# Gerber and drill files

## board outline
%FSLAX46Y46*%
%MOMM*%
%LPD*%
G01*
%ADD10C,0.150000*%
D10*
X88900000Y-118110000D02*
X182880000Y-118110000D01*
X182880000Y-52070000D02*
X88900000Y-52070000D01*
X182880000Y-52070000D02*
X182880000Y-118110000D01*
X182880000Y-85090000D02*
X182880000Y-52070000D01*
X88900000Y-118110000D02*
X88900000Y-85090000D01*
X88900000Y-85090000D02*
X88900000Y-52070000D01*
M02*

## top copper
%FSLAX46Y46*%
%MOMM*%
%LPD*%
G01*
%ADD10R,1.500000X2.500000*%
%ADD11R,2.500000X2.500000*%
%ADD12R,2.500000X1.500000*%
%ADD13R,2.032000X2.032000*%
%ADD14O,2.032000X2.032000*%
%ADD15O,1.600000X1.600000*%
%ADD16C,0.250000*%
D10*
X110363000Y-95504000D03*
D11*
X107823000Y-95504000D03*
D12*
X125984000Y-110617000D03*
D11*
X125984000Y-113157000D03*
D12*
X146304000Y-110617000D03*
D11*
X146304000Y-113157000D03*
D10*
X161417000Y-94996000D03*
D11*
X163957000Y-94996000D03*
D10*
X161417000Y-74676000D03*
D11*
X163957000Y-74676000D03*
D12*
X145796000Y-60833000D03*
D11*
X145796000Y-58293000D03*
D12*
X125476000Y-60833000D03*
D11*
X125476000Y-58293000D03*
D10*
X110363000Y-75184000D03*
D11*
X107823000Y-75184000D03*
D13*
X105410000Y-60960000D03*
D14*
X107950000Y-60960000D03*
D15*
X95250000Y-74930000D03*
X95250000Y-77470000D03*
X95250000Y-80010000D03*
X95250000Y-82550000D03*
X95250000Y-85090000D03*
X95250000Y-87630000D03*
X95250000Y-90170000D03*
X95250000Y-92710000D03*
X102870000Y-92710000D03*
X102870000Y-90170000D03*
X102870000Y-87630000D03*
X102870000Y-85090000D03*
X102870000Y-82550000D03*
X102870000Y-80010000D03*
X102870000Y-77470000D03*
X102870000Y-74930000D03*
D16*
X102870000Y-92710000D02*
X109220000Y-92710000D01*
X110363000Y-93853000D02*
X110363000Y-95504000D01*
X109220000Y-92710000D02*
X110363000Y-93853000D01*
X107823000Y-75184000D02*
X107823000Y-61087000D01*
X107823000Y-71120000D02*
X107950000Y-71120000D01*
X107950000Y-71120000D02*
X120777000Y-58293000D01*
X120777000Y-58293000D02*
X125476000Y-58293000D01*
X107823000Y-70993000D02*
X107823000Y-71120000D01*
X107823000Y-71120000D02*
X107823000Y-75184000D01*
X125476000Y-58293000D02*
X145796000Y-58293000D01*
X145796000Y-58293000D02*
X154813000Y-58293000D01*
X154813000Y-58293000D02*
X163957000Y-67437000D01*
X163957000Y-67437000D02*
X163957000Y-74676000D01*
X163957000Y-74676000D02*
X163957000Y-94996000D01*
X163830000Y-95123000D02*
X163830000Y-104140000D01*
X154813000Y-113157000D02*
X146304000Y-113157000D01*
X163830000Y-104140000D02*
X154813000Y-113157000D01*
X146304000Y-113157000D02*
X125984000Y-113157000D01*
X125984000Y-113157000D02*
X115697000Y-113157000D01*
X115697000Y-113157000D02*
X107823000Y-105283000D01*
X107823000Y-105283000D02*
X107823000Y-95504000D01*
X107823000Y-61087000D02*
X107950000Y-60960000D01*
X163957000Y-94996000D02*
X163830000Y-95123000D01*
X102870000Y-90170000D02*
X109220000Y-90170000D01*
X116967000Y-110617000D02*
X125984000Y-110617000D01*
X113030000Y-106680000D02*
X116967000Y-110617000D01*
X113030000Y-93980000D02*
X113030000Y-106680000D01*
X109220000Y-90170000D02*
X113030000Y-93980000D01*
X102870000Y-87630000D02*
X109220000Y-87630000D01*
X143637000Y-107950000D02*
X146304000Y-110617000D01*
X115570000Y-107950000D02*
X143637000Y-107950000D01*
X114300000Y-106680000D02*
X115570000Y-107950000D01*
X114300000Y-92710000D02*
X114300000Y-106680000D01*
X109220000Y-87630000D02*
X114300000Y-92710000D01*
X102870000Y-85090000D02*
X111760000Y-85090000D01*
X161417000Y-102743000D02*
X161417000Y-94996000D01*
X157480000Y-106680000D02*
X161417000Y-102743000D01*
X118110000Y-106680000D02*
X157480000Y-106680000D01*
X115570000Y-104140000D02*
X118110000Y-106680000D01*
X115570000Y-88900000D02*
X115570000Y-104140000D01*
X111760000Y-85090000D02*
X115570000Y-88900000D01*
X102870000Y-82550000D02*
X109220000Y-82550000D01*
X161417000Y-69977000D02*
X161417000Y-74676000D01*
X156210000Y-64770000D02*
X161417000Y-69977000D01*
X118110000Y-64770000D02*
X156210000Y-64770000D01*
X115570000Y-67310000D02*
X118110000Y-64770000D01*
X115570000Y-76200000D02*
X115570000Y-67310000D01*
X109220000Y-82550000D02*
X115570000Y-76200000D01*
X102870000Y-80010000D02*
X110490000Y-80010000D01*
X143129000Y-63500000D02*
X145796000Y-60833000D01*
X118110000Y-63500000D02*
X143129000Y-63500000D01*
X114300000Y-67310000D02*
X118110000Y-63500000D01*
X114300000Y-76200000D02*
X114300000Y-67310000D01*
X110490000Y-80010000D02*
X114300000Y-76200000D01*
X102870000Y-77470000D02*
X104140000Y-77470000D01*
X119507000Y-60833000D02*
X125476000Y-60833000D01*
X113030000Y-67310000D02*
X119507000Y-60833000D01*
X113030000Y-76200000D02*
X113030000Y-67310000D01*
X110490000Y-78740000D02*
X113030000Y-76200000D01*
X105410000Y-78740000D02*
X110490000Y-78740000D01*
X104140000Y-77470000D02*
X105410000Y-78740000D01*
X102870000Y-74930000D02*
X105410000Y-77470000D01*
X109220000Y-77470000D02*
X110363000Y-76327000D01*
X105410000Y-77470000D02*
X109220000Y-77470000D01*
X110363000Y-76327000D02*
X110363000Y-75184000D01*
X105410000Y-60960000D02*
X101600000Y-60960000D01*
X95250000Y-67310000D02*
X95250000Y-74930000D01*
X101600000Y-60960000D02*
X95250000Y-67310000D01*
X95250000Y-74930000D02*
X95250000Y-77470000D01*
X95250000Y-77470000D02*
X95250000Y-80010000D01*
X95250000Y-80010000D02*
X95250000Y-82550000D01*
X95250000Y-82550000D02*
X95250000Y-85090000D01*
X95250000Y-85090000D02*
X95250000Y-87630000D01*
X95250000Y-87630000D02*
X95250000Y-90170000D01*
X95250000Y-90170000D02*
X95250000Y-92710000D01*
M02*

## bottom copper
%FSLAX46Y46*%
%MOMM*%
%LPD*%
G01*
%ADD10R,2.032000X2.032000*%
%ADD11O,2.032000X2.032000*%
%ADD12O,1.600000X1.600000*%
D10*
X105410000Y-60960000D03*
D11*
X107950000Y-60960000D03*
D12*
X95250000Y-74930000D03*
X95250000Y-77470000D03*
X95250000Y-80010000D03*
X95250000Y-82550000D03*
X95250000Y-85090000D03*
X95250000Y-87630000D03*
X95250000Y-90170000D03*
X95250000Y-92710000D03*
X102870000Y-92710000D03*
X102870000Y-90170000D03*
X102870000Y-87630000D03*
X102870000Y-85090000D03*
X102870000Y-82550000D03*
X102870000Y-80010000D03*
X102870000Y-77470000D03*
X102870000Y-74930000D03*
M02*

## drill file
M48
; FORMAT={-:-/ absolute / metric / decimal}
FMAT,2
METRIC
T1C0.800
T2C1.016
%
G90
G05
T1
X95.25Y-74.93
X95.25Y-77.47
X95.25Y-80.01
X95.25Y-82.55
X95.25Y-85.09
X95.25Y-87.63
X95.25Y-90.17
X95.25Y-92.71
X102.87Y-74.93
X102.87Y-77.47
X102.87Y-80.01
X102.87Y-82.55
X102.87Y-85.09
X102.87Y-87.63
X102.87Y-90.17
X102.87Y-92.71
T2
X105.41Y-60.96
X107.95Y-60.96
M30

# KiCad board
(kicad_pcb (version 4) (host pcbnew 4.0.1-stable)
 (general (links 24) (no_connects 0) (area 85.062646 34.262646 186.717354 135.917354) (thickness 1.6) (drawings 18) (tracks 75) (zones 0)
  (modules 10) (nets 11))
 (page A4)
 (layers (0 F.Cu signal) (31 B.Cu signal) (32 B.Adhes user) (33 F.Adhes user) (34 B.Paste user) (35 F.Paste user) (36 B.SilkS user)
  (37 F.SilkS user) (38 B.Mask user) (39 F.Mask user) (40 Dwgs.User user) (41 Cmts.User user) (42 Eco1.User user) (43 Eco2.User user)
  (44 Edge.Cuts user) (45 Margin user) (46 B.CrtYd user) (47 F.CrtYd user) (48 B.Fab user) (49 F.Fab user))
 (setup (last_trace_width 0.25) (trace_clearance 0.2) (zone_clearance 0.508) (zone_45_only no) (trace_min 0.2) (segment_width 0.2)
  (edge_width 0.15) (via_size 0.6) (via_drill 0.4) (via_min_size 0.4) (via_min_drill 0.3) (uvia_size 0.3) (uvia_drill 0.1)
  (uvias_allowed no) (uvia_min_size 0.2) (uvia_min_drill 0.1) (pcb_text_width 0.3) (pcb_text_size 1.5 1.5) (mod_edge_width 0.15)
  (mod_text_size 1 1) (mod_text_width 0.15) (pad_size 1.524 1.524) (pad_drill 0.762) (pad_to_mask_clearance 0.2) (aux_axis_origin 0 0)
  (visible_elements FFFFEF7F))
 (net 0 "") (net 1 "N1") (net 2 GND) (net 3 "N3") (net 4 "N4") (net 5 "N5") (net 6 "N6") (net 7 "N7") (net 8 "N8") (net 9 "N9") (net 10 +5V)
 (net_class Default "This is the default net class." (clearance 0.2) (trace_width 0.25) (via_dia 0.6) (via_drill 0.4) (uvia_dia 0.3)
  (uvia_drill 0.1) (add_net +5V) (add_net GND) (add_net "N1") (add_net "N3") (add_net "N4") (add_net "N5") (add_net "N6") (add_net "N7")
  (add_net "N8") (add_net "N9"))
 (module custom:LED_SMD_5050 (layer F.Cu) (at 109.22 91.44)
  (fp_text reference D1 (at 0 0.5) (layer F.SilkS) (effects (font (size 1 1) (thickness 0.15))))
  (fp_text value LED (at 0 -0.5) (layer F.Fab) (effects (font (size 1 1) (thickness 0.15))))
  (pad 2 smd rect (at 1.143 4.064) (size 1.5 2.5) (layers F.Cu F.Paste F.Mask) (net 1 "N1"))
  (pad 1 smd rect (at -1.397 4.064) (size 2.5 2.5) (layers F.Cu F.Paste F.Mask) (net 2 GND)))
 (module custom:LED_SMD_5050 (layer F.Cu) (at 121.92 111.76 90)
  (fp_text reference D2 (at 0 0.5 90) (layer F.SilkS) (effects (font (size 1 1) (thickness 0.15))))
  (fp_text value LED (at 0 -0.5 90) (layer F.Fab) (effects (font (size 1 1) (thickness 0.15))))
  (pad 2 smd rect (at 1.143 4.064 90) (size 1.5 2.5) (layers F.Cu F.Paste F.Mask) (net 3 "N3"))
  (pad 1 smd rect (at -1.397 4.064 90) (size 2.5 2.5) (layers F.Cu F.Paste F.Mask) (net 2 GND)))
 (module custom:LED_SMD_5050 (layer F.Cu) (at 142.24 111.76 90)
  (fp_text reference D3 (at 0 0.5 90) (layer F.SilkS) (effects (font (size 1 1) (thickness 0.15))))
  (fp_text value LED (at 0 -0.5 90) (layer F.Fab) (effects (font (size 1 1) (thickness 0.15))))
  (pad 2 smd rect (at 1.143 4.064 90) (size 1.5 2.5) (layers F.Cu F.Paste F.Mask) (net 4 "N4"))
  (pad 1 smd rect (at -1.397 4.064 90) (size 2.5 2.5) (layers F.Cu F.Paste F.Mask) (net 2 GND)))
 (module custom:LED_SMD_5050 (layer F.Cu) (at 162.56 99.06 180)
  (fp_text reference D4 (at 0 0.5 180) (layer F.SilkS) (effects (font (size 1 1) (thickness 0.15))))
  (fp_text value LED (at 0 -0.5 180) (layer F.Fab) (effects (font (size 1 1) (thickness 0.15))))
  (pad 2 smd rect (at 1.143 4.064 180) (size 1.5 2.5) (layers F.Cu F.Paste F.Mask) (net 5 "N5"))
  (pad 1 smd rect (at -1.397 4.064 180) (size 2.5 2.5) (layers F.Cu F.Paste F.Mask) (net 2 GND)))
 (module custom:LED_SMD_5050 (layer F.Cu) (at 162.56 78.74 180)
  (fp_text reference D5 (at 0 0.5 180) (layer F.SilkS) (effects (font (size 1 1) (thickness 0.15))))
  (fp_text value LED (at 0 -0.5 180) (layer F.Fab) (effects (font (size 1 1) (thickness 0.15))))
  (pad 2 smd rect (at 1.143 4.064 180) (size 1.5 2.5) (layers F.Cu F.Paste F.Mask) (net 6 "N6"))
  (pad 1 smd rect (at -1.397 4.064 180) (size 2.5 2.5) (layers F.Cu F.Paste F.Mask) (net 2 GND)))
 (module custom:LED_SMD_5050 (layer F.Cu) (at 149.86 59.69 270)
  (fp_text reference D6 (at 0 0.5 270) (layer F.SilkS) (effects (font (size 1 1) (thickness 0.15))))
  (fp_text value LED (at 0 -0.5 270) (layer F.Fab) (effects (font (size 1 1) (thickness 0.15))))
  (pad 2 smd rect (at 1.143 4.064 270) (size 1.5 2.5) (layers F.Cu F.Paste F.Mask) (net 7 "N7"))
  (pad 1 smd rect (at -1.397 4.064 270) (size 2.5 2.5) (layers F.Cu F.Paste F.Mask) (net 2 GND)))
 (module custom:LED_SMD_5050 (layer F.Cu) (at 129.54 59.69 270)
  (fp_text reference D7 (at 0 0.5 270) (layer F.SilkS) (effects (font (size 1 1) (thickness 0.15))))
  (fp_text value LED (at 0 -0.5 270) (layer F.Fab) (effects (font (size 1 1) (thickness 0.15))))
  (pad 2 smd rect (at 1.143 4.064 270) (size 1.5 2.5) (layers F.Cu F.Paste F.Mask) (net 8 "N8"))
  (pad 1 smd rect (at -1.397 4.064 270) (size 2.5 2.5) (layers F.Cu F.Paste F.Mask) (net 2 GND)))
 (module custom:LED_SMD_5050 (layer F.Cu) (at 109.22 71.12)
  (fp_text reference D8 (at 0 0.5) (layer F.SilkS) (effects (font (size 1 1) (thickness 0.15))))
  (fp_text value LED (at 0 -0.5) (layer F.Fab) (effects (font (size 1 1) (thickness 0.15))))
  (pad 2 smd rect (at 1.143 4.064) (size 1.5 2.5) (layers F.Cu F.Paste F.Mask) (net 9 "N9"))
  (pad 1 smd rect (at -1.397 4.064) (size 2.5 2.5) (layers F.Cu F.Paste F.Mask) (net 2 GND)))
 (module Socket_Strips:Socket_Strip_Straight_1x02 (layer F.Cu) (at 105.41 60.96)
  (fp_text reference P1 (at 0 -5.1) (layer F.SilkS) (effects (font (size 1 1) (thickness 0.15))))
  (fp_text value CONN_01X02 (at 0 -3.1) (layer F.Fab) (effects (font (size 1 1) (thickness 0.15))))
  (pad 1 thru_hole rect (at 0 0) (size 2.032 2.032) (drill 1.016) (layers *.Cu *.Mask F.SilkS) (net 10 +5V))
  (pad 2 thru_hole oval (at 2.54 0) (size 2.032 2.032) (drill 1.016) (layers *.Cu *.Mask F.SilkS) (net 2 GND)))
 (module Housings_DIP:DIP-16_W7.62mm (layer F.Cu) (at 95.25 74.93)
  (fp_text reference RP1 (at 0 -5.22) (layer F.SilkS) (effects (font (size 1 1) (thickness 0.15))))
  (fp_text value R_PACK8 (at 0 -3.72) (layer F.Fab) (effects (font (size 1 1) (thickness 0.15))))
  (pad 1 thru_hole oval (at 0 0) (size 1.6 1.6) (drill 0.8) (layers *.Cu *.Mask F.SilkS) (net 10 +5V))
  (pad 2 thru_hole oval (at 0 2.54) (size 1.6 1.6) (drill 0.8) (layers *.Cu *.Mask F.SilkS) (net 10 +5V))
  (pad 3 thru_hole oval (at 0 5.08) (size 1.6 1.6) (drill 0.8) (layers *.Cu *.Mask F.SilkS) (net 10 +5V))
  (pad 4 thru_hole oval (at 0 7.62) (size 1.6 1.6) (drill 0.8) (layers *.Cu *.Mask F.SilkS) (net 10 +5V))
  (pad 5 thru_hole oval (at 0 10.16) (size 1.6 1.6) (drill 0.8) (layers *.Cu *.Mask F.SilkS) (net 10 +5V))
  (pad 6 thru_hole oval (at 0 12.7) (size 1.6 1.6) (drill 0.8) (layers *.Cu *.Mask F.SilkS) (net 10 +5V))
  (pad 7 thru_hole oval (at 0 15.24) (size 1.6 1.6) (drill 0.8) (layers *.Cu *.Mask F.SilkS) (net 10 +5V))
  (pad 8 thru_hole oval (at 0 17.78) (size 1.6 1.6) (drill 0.8) (layers *.Cu *.Mask F.SilkS) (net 10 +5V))
  (pad 9 thru_hole oval (at 7.62 17.78) (size 1.6 1.6) (drill 0.8) (layers *.Cu *.Mask F.SilkS) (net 1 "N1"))
  (pad 10 thru_hole oval (at 7.62 15.24) (size 1.6 1.6) (drill 0.8) (layers *.Cu *.Mask F.SilkS) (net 3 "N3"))
  (pad 11 thru_hole oval (at 7.62 12.7) (size 1.6 1.6) (drill 0.8) (layers *.Cu *.Mask F.SilkS) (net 4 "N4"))
  (pad 12 thru_hole oval (at 7.62 10.16) (size 1.6 1.6) (drill 0.8) (layers *.Cu *.Mask F.SilkS) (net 5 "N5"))
  (pad 13 thru_hole oval (at 7.62 7.62) (size 1.6 1.6) (drill 0.8) (layers *.Cu *.Mask F.SilkS) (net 6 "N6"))
  (pad 14 thru_hole oval (at 7.62 5.08) (size 1.6 1.6) (drill 0.8) (layers *.Cu *.Mask F.SilkS) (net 7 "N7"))
  (pad 15 thru_hole oval (at 7.62 2.54) (size 1.6 1.6) (drill 0.8) (layers *.Cu *.Mask F.SilkS) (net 8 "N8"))
  (pad 16 thru_hole oval (at 7.62 0) (size 1.6 1.6) (drill 0.8) (layers *.Cu *.Mask F.SilkS) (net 9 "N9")))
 (gr_line (start 88.9 118.11) (end 182.88 118.11) (angle 90) (layer Edge.Cuts) (width 0.15))
 (gr_line (start 182.88 52.07) (end 88.9 52.07) (angle 90) (layer Edge.Cuts) (width 0.15))
 (gr_line (start 182.88 52.07) (end 182.88 118.11) (angle 90) (layer Edge.Cuts) (width 0.15))
 (gr_line (start 182.88 85.09) (end 182.88 52.07) (angle 90) (layer Edge.Cuts) (width 0.15))
 (gr_line (start 88.9 118.11) (end 88.9 85.09) (angle 90) (layer Edge.Cuts) (width 0.15))
 (gr_line (start 88.9 85.09) (end 88.9 52.07) (angle 90) (layer Edge.Cuts) (width 0.15))
 (segment (start 102.87 92.71) (end 109.22 92.71) (width 0.25) (layer F.Cu) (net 1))
 (segment (start 110.363 93.853) (end 110.363 95.504) (width 0.25) (layer F.Cu) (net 1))
 (segment (start 109.22 92.71) (end 110.363 93.853) (width 0.25) (layer F.Cu) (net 1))
 (segment (start 107.823 75.184) (end 107.823 61.087) (width 0.25) (layer F.Cu) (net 2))
 (segment (start 107.823 71.12) (end 107.95 71.12) (width 0.25) (layer F.Cu) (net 2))
 (segment (start 107.95 71.12) (end 120.777 58.293) (width 0.25) (layer F.Cu) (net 2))
 (segment (start 120.777 58.293) (end 125.476 58.293) (width 0.25) (layer F.Cu) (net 2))
 (segment (start 107.823 70.993) (end 107.823 71.12) (width 0.25) (layer F.Cu) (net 2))
 (segment (start 107.823 71.12) (end 107.823 75.184) (width 0.25) (layer F.Cu) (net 2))
 (segment (start 125.476 58.293) (end 145.796 58.293) (width 0.25) (layer F.Cu) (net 2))
 (segment (start 145.796 58.293) (end 154.813 58.293) (width 0.25) (layer F.Cu) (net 2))
 (segment (start 154.813 58.293) (end 163.957 67.437) (width 0.25) (layer F.Cu) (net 2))
 (segment (start 163.957 67.437) (end 163.957 74.676) (width 0.25) (layer F.Cu) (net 2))
 (segment (start 163.957 74.676) (end 163.957 94.996) (width 0.25) (layer F.Cu) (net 2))
 (segment (start 163.83 95.123) (end 163.83 104.14) (width 0.25) (layer F.Cu) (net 2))
 (segment (start 154.813 113.157) (end 146.304 113.157) (width 0.25) (layer F.Cu) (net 2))
 (segment (start 163.83 104.14) (end 154.813 113.157) (width 0.25) (layer F.Cu) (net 2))
 (segment (start 146.304 113.157) (end 125.984 113.157) (width 0.25) (layer F.Cu) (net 2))
 (segment (start 125.984 113.157) (end 115.697 113.157) (width 0.25) (layer F.Cu) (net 2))
 (segment (start 115.697 113.157) (end 107.823 105.283) (width 0.25) (layer F.Cu) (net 2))
 (segment (start 107.823 105.283) (end 107.823 95.504) (width 0.25) (layer F.Cu) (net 2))
 (segment (start 107.823 61.087) (end 107.95 60.96) (width 0.25) (layer F.Cu) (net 2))
 (segment (start 163.957 94.996) (end 163.83 95.123) (width 0.25) (layer F.Cu) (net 2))
 (segment (start 102.87 90.17) (end 109.22 90.17) (width 0.25) (layer F.Cu) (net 3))
 (segment (start 116.967 110.617) (end 125.984 110.617) (width 0.25) (layer F.Cu) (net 3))
 (segment (start 113.03 106.68) (end 116.967 110.617) (width 0.25) (layer F.Cu) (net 3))
 (segment (start 113.03 93.98) (end 113.03 106.68) (width 0.25) (layer F.Cu) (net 3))
 (segment (start 109.22 90.17) (end 113.03 93.98) (width 0.25) (layer F.Cu) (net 3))
 (segment (start 102.87 87.63) (end 109.22 87.63) (width 0.25) (layer F.Cu) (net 4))
 (segment (start 143.637 107.95) (end 146.304 110.617) (width 0.25) (layer F.Cu) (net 4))
 (segment (start 115.57 107.95) (end 143.637 107.95) (width 0.25) (layer F.Cu) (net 4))
 (segment (start 114.3 106.68) (end 115.57 107.95) (width 0.25) (layer F.Cu) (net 4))
 (segment (start 114.3 92.71) (end 114.3 106.68) (width 0.25) (layer F.Cu) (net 4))
 (segment (start 109.22 87.63) (end 114.3 92.71) (width 0.25) (layer F.Cu) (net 4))
 (segment (start 102.87 85.09) (end 111.76 85.09) (width 0.25) (layer F.Cu) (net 5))
 (segment (start 161.417 102.743) (end 161.417 94.996) (width 0.25) (layer F.Cu) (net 5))
 (segment (start 157.48 106.68) (end 161.417 102.743) (width 0.25) (layer F.Cu) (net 5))
 (segment (start 118.11 106.68) (end 157.48 106.68) (width 0.25) (layer F.Cu) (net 5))
 (segment (start 115.57 104.14) (end 118.11 106.68) (width 0.25) (layer F.Cu) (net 5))
 (segment (start 115.57 88.9) (end 115.57 104.14) (width 0.25) (layer F.Cu) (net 5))
 (segment (start 111.76 85.09) (end 115.57 88.9) (width 0.25) (layer F.Cu) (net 5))
 (segment (start 102.87 82.55) (end 109.22 82.55) (width 0.25) (layer F.Cu) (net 6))
 (segment (start 161.417 69.977) (end 161.417 74.676) (width 0.25) (layer F.Cu) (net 6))
 (segment (start 156.21 64.77) (end 161.417 69.977) (width 0.25) (layer F.Cu) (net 6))
 (segment (start 118.11 64.77) (end 156.21 64.77) (width 0.25) (layer F.Cu) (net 6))
 (segment (start 115.57 67.31) (end 118.11 64.77) (width 0.25) (layer F.Cu) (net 6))
 (segment (start 115.57 76.2) (end 115.57 67.31) (width 0.25) (layer F.Cu) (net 6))
 (segment (start 109.22 82.55) (end 115.57 76.2) (width 0.25) (layer F.Cu) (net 6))
 (segment (start 102.87 80.01) (end 110.49 80.01) (width 0.25) (layer F.Cu) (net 7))
 (segment (start 143.129 63.5) (end 145.796 60.833) (width 0.25) (layer F.Cu) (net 7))
 (segment (start 118.11 63.5) (end 143.129 63.5) (width 0.25) (layer F.Cu) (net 7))
 (segment (start 114.3 67.31) (end 118.11 63.5) (width 0.25) (layer F.Cu) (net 7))
 (segment (start 114.3 76.2) (end 114.3 67.31) (width 0.25) (layer F.Cu) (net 7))
 (segment (start 110.49 80.01) (end 114.3 76.2) (width 0.25) (layer F.Cu) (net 7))
 (segment (start 102.87 77.47) (end 104.14 77.47) (width 0.25) (layer F.Cu) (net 8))
 (segment (start 119.507 60.833) (end 125.476 60.833) (width 0.25) (layer F.Cu) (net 8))
 (segment (start 113.03 67.31) (end 119.507 60.833) (width 0.25) (layer F.Cu) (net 8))
 (segment (start 113.03 76.2) (end 113.03 67.31) (width 0.25) (layer F.Cu) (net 8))
 (segment (start 110.49 78.74) (end 113.03 76.2) (width 0.25) (layer F.Cu) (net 8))
 (segment (start 105.41 78.74) (end 110.49 78.74) (width 0.25) (layer F.Cu) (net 8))
 (segment (start 104.14 77.47) (end 105.41 78.74) (width 0.25) (layer F.Cu) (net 8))
 (segment (start 102.87 74.93) (end 105.41 77.47) (width 0.25) (layer F.Cu) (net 9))
 (segment (start 109.22 77.47) (end 110.363 76.327) (width 0.25) (layer F.Cu) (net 9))
 (segment (start 105.41 77.47) (end 109.22 77.47) (width 0.25) (layer F.Cu) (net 9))
 (segment (start 110.363 76.327) (end 110.363 75.184) (width 0.25) (layer F.Cu) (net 9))
 (segment (start 105.41 60.96) (end 101.6 60.96) (width 0.25) (layer F.Cu) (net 10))
 (segment (start 95.25 67.31) (end 95.25 74.93) (width 0.25) (layer F.Cu) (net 10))
 (segment (start 101.6 60.96) (end 95.25 67.31) (width 0.25) (layer F.Cu) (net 10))
 (segment (start 95.25 74.93) (end 95.25 77.47) (width 0.25) (layer F.Cu) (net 10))
 (segment (start 95.25 77.47) (end 95.25 80.01) (width 0.25) (layer F.Cu) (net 10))
 (segment (start 95.25 80.01) (end 95.25 82.55) (width 0.25) (layer F.Cu) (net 10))
 (segment (start 95.25 82.55) (end 95.25 85.09) (width 0.25) (layer F.Cu) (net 10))
 (segment (start 95.25 85.09) (end 95.25 87.63) (width 0.25) (layer F.Cu) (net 10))
 (segment (start 95.25 87.63) (end 95.25 90.17) (width 0.25) (layer F.Cu) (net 10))
 (segment (start 95.25 90.17) (end 95.25 92.71) (width 0.25) (layer F.Cu) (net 10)))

